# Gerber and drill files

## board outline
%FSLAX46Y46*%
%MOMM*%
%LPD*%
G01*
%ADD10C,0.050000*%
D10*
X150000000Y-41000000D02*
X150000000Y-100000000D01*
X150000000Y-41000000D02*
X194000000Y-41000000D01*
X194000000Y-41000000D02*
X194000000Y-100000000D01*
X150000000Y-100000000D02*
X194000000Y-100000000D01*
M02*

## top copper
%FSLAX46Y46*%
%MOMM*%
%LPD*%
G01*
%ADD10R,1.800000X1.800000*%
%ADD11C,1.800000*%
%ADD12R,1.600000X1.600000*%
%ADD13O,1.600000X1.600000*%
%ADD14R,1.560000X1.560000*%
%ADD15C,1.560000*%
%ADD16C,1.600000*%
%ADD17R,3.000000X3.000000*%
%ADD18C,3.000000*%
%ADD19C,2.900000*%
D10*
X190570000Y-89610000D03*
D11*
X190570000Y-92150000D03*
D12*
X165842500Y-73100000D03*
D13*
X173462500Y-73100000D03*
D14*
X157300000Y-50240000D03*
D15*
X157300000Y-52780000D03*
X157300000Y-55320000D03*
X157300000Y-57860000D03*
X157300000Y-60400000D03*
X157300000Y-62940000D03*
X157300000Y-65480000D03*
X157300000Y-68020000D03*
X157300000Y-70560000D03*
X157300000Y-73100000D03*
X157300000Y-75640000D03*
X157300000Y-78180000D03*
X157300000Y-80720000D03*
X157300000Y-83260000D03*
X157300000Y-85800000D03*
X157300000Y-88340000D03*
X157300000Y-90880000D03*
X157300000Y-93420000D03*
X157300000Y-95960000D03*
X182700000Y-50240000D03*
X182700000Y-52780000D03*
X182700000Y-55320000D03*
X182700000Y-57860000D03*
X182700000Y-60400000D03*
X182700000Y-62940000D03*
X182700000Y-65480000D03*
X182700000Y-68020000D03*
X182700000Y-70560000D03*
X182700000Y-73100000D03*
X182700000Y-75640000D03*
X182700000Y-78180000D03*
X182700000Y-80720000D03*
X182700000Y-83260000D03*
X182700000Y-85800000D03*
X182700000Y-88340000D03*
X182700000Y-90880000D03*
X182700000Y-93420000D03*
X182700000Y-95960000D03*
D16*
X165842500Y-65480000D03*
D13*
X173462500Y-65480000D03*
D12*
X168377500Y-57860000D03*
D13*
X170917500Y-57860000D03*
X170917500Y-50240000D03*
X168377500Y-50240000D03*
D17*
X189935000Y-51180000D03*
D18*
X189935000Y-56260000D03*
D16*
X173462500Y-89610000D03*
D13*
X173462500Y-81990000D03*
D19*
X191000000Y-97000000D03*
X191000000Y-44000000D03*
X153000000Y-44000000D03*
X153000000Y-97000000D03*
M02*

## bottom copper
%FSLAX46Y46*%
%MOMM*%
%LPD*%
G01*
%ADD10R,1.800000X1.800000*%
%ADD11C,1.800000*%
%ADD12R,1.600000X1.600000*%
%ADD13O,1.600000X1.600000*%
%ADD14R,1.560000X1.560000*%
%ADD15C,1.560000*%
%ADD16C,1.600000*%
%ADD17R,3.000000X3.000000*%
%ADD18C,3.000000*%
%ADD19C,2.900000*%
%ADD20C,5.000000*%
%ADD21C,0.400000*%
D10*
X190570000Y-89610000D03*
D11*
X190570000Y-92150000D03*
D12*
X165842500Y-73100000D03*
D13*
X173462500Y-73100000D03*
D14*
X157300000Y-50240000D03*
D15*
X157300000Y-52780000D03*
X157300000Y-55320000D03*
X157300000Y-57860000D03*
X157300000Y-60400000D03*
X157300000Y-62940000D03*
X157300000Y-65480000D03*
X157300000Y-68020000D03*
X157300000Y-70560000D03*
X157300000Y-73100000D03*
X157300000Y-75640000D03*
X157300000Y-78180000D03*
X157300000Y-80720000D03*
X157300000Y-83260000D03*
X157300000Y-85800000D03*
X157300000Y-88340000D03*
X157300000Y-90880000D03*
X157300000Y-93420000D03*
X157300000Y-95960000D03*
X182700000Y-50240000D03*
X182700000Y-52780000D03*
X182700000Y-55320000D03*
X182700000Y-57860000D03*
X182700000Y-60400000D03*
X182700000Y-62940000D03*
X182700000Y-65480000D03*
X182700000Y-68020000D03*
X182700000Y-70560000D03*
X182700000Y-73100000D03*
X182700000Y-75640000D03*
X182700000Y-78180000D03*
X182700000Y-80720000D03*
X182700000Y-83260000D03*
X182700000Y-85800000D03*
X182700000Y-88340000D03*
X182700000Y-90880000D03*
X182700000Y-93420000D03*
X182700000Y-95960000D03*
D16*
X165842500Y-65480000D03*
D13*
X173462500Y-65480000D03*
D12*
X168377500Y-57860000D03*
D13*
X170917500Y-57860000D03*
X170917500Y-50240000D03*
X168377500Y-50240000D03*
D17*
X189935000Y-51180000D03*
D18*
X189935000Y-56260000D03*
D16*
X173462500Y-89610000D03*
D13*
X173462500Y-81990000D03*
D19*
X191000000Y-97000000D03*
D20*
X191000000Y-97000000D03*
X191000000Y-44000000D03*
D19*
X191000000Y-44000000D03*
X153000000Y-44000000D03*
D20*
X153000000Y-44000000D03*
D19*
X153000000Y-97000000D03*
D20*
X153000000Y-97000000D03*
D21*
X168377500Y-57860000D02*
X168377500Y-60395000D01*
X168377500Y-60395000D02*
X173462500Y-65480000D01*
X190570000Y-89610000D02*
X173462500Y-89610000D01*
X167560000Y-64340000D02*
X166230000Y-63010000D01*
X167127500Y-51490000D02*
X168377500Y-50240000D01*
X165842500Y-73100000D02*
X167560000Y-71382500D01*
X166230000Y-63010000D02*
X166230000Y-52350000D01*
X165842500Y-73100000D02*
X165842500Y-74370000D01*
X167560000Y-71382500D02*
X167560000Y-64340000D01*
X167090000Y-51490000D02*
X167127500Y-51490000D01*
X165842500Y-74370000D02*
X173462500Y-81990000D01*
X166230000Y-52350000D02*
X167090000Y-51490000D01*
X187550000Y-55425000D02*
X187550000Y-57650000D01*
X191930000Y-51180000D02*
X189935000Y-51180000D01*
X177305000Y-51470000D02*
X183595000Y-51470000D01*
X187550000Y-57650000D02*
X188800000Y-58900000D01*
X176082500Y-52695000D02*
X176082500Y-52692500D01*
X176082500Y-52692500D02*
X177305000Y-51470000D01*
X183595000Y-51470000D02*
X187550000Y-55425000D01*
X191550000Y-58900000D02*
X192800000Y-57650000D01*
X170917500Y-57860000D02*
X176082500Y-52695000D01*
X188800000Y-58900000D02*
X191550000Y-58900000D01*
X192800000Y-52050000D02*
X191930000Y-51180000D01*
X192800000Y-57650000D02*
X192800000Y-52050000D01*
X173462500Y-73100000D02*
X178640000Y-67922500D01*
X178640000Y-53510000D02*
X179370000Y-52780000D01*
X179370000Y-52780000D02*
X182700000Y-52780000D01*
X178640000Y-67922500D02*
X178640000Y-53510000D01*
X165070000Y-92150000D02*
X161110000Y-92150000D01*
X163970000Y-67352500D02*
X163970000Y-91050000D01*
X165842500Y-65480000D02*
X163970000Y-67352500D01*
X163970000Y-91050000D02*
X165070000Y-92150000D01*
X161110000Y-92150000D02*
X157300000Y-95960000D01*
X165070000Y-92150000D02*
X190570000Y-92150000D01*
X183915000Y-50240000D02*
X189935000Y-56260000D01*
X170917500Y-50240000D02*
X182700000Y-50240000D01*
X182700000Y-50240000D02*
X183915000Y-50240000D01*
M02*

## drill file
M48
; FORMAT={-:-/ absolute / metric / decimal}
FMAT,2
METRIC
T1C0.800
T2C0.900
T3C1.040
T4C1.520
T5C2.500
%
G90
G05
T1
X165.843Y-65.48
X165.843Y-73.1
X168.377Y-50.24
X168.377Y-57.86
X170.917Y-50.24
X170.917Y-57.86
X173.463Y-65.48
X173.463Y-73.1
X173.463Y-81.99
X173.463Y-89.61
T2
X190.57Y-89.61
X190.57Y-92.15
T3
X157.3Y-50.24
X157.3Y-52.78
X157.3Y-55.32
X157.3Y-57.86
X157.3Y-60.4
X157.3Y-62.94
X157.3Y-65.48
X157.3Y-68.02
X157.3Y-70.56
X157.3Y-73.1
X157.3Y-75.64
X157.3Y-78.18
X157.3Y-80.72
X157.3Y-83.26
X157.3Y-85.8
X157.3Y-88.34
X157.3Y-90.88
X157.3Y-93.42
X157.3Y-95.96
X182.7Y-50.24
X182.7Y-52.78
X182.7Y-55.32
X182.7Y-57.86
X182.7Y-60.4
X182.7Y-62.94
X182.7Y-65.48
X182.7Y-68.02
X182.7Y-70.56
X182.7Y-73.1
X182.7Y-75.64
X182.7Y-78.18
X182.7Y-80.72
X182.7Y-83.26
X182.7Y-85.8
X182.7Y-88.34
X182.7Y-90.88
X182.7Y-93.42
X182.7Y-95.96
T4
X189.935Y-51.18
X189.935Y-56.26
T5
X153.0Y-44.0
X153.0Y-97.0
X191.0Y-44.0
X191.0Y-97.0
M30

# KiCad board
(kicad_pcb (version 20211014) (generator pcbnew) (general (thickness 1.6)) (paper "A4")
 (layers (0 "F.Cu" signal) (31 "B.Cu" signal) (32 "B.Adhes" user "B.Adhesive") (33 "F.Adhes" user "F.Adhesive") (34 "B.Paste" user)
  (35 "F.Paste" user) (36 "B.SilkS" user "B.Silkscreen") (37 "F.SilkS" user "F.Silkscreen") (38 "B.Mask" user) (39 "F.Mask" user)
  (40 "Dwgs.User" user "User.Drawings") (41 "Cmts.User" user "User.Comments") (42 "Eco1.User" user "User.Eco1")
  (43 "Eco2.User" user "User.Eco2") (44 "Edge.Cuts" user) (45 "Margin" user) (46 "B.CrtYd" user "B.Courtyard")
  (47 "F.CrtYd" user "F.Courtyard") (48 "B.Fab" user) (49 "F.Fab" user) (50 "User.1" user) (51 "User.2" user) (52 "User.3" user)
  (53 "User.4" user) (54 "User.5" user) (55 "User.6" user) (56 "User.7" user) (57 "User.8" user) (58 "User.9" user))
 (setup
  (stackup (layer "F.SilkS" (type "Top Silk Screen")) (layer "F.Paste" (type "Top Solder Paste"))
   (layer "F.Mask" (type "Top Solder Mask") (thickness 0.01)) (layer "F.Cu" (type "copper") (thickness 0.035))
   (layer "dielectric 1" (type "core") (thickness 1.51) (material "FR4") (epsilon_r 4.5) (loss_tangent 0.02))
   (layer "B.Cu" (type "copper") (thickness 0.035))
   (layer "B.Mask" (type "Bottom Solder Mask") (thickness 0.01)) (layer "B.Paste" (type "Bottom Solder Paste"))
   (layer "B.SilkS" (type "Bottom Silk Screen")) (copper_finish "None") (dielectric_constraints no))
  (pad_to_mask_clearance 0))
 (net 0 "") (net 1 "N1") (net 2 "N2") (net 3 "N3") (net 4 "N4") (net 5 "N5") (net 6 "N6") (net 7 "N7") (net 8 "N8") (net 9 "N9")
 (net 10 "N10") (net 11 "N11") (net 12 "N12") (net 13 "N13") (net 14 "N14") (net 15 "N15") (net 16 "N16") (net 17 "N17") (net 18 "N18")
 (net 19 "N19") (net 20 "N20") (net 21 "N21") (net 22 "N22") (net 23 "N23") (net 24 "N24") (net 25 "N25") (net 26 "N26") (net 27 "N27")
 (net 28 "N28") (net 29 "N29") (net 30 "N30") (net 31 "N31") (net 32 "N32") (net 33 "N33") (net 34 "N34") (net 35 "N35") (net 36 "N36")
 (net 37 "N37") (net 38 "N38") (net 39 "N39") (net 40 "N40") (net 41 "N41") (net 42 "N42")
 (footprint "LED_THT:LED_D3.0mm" (layer "F.Cu") (at 190.57 89.61 -90)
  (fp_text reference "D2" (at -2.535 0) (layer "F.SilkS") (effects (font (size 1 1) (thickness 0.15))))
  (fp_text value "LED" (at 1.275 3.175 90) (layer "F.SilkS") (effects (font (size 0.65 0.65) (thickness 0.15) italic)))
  (pad "1" thru_hole rect (at 0 0 270) (size 1.8 1.8) (drill 0.9) (layers *.Cu *.Mask) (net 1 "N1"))
  (pad "2" thru_hole circle (at 2.54 0 270) (size 1.8 1.8) (drill 0.9) (layers *.Cu *.Mask) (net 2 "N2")))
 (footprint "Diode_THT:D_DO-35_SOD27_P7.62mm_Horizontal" (layer "F.Cu") (at 165.8425 73.1)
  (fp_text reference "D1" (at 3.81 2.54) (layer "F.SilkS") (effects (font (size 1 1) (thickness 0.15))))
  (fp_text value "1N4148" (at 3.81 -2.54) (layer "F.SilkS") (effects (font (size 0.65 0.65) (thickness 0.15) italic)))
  (pad "1" thru_hole rect (at 0 0) (size 1.6 1.6) (drill 0.8) (layers *.Cu *.Mask) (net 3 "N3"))
  (pad "2" thru_hole oval (at 7.62 0) (size 1.6 1.6) (drill 0.8) (layers *.Cu *.Mask) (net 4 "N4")))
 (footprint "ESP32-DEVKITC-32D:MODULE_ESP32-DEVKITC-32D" (layer "F.Cu") (at 170 70)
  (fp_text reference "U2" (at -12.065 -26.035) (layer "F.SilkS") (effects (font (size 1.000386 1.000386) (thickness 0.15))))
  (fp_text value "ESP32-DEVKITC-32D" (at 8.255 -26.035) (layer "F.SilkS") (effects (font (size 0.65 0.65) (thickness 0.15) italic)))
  (pad "1" thru_hole rect locked (at -12.7 -19.76) (size 1.56 1.56) (drill 1.04) (layers *.Cu *.Mask) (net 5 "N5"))
  (pad "2" thru_hole circle locked (at -12.7 -17.22) (size 1.56 1.56) (drill 1.04) (layers *.Cu *.Mask) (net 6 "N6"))
  (pad "3" thru_hole circle locked (at -12.7 -14.68) (size 1.56 1.56) (drill 1.04) (layers *.Cu *.Mask) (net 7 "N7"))
  (pad "4" thru_hole circle locked (at -12.7 -12.14) (size 1.56 1.56) (drill 1.04) (layers *.Cu *.Mask) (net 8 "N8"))
  (pad "5" thru_hole circle locked (at -12.7 -9.6) (size 1.56 1.56) (drill 1.04) (layers *.Cu *.Mask) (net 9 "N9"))
  (pad "6" thru_hole circle locked (at -12.7 -7.06) (size 1.56 1.56) (drill 1.04) (layers *.Cu *.Mask) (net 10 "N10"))
  (pad "7" thru_hole circle locked (at -12.7 -4.52) (size 1.56 1.56) (drill 1.04) (layers *.Cu *.Mask) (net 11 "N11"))
  (pad "8" thru_hole circle locked (at -12.7 -1.98) (size 1.56 1.56) (drill 1.04) (layers *.Cu *.Mask) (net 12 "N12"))
  (pad "9" thru_hole circle locked (at -12.7 0.56) (size 1.56 1.56) (drill 1.04) (layers *.Cu *.Mask) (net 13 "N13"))
  (pad "10" thru_hole circle locked (at -12.7 3.1) (size 1.56 1.56) (drill 1.04) (layers *.Cu *.Mask) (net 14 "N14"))
  (pad "11" thru_hole circle locked (at -12.7 5.64) (size 1.56 1.56) (drill 1.04) (layers *.Cu *.Mask) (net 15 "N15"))
  (pad "12" thru_hole circle locked (at -12.7 8.18) (size 1.56 1.56) (drill 1.04) (layers *.Cu *.Mask) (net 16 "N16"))
  (pad "13" thru_hole circle locked (at -12.7 10.72) (size 1.56 1.56) (drill 1.04) (layers *.Cu *.Mask) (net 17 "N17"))
  (pad "14" thru_hole circle locked (at -12.7 13.26) (size 1.56 1.56) (drill 1.04) (layers *.Cu *.Mask) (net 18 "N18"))
  (pad "15" thru_hole circle locked (at -12.7 15.8) (size 1.56 1.56) (drill 1.04) (layers *.Cu *.Mask) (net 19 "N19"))
  (pad "16" thru_hole circle locked (at -12.7 18.34) (size 1.56 1.56) (drill 1.04) (layers *.Cu *.Mask) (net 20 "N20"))
  (pad "17" thru_hole circle locked (at -12.7 20.88) (size 1.56 1.56) (drill 1.04) (layers *.Cu *.Mask) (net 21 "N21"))
  (pad "18" thru_hole circle locked (at -12.7 23.42) (size 1.56 1.56) (drill 1.04) (layers *.Cu *.Mask) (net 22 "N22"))
  (pad "19" thru_hole circle locked (at -12.7 25.96) (size 1.56 1.56) (drill 1.04) (layers *.Cu *.Mask) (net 2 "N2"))
  (pad "20" thru_hole circle locked (at 12.7 -19.76) (size 1.56 1.56) (drill 1.04) (layers *.Cu *.Mask) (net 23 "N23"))
  (pad "21" thru_hole circle locked (at 12.7 -17.22) (size 1.56 1.56) (drill 1.04) (layers *.Cu *.Mask) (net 4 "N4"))
  (pad "22" thru_hole circle locked (at 12.7 -14.68) (size 1.56 1.56) (drill 1.04) (layers *.Cu *.Mask) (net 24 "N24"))
  (pad "23" thru_hole circle locked (at 12.7 -12.14) (size 1.56 1.56) (drill 1.04) (layers *.Cu *.Mask) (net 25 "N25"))
  (pad "24" thru_hole circle locked (at 12.7 -9.6) (size 1.56 1.56) (drill 1.04) (layers *.Cu *.Mask) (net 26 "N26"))
  (pad "25" thru_hole circle locked (at 12.7 -7.06) (size 1.56 1.56) (drill 1.04) (layers *.Cu *.Mask) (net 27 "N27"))
  (pad "26" thru_hole circle locked (at 12.7 -4.52) (size 1.56 1.56) (drill 1.04) (layers *.Cu *.Mask) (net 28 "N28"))
  (pad "27" thru_hole circle locked (at 12.7 -1.98) (size 1.56 1.56) (drill 1.04) (layers *.Cu *.Mask) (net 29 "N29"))
  (pad "28" thru_hole circle locked (at 12.7 0.56) (size 1.56 1.56) (drill 1.04) (layers *.Cu *.Mask) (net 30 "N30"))
  (pad "29" thru_hole circle locked (at 12.7 3.1) (size 1.56 1.56) (drill 1.04) (layers *.Cu *.Mask) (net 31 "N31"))
  (pad "30" thru_hole circle locked (at 12.7 5.64) (size 1.56 1.56) (drill 1.04) (layers *.Cu *.Mask) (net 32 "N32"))
  (pad "31" thru_hole circle locked (at 12.7 8.18) (size 1.56 1.56) (drill 1.04) (layers *.Cu *.Mask) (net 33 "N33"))
  (pad "32" thru_hole circle locked (at 12.7 10.72) (size 1.56 1.56) (drill 1.04) (layers *.Cu *.Mask) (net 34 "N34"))
  (pad "33" thru_hole circle locked (at 12.7 13.26) (size 1.56 1.56) (drill 1.04) (layers *.Cu *.Mask) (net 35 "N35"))
  (pad "34" thru_hole circle locked (at 12.7 15.8) (size 1.56 1.56) (drill 1.04) (layers *.Cu *.Mask) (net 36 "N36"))
  (pad "35" thru_hole circle locked (at 12.7 18.34) (size 1.56 1.56) (drill 1.04) (layers *.Cu *.Mask) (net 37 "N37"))
  (pad "36" thru_hole circle locked (at 12.7 20.88) (size 1.56 1.56) (drill 1.04) (layers *.Cu *.Mask) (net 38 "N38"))
  (pad "37" thru_hole circle locked (at 12.7 23.42) (size 1.56 1.56) (drill 1.04) (layers *.Cu *.Mask) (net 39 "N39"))
  (pad "38" thru_hole circle locked (at 12.7 25.96) (size 1.56 1.56) (drill 1.04) (layers *.Cu *.Mask) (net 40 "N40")))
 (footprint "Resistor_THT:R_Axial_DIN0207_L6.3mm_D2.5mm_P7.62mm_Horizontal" (layer "F.Cu") (at 165.8425 65.48)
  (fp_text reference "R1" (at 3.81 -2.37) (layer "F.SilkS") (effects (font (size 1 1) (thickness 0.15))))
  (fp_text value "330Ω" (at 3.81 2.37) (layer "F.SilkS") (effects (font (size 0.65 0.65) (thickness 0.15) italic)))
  (pad "1" thru_hole circle (at 0 0) (size 1.6 1.6) (drill 0.8) (layers *.Cu *.Mask) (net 2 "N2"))
  (pad "2" thru_hole oval (at 7.62 0) (size 1.6 1.6) (drill 0.8) (layers *.Cu *.Mask) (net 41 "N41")))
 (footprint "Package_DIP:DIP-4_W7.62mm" (layer "F.Cu") (at 168.3775 57.86 90)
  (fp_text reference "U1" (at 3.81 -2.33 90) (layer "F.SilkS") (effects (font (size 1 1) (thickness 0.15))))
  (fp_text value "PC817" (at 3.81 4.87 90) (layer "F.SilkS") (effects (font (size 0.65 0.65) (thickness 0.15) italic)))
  (pad "1" thru_hole rect (at 0 0 90) (size 1.6 1.6) (drill 0.8) (layers *.Cu *.Mask) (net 41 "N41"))
  (pad "2" thru_hole oval (at 0 2.54 90) (size 1.6 1.6) (drill 0.8) (layers *.Cu *.Mask) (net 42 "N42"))
  (pad "3" thru_hole oval (at 7.62 2.54 90) (size 1.6 1.6) (drill 0.8) (layers *.Cu *.Mask) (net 23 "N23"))
  (pad "4" thru_hole oval (at 7.62 0 90) (size 1.6 1.6) (drill 0.8) (layers *.Cu *.Mask) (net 3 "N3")))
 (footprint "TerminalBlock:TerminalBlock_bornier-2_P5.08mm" (layer "F.Cu") (at 189.935 51.18 -90)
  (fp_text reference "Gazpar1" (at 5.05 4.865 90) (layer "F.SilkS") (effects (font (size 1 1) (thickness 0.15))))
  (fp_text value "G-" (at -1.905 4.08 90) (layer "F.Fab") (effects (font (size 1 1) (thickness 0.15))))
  (pad "1" thru_hole rect (at 0 0 270) (size 3 3) (drill 1.52) (layers *.Cu *.Mask) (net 42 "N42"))
  (pad "2" thru_hole circle (at 5.08 0 270) (size 3 3) (drill 1.52) (layers *.Cu *.Mask) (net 23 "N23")))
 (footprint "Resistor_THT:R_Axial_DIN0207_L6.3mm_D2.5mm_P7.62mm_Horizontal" (layer "F.Cu") (at 173.4625 89.61 90)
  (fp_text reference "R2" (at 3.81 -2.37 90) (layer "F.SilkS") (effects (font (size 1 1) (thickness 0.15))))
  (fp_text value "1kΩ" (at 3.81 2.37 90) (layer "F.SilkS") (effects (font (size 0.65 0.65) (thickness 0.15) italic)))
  (pad "1" thru_hole circle (at 0 0 90) (size 1.6 1.6) (drill 0.8) (layers *.Cu *.Mask) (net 1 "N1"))
  (pad "2" thru_hole oval (at 7.62 0 90) (size 1.6 1.6) (drill 0.8) (layers *.Cu *.Mask) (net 3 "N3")))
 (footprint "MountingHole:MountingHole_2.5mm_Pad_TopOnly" (layer "B.Cu") (at 191 97 180)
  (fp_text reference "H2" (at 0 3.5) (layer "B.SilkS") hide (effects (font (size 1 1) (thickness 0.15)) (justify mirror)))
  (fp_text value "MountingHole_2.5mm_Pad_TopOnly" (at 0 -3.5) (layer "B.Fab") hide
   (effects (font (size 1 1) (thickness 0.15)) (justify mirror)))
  (pad "1" thru_hole circle (at 0 0 180) (size 2.9 2.9) (drill 2.5) (layers *.Cu *.Mask))
  (pad "1" connect circle (at 0 0 180) (size 5 5) (layers "B.Cu" "B.Mask")))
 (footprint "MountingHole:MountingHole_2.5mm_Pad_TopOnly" (layer "B.Cu") (at 191 44 180)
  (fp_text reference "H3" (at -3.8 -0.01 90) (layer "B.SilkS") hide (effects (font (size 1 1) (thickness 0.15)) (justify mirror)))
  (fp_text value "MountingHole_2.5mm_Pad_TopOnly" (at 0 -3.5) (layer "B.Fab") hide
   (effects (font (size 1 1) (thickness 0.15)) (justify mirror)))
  (pad "1" connect circle (at 0 0 180) (size 5 5) (layers "B.Cu" "B.Mask"))
  (pad "1" thru_hole circle (at 0 0 180) (size 2.9 2.9) (drill 2.5) (layers *.Cu *.Mask)))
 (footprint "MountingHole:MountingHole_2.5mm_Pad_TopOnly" (layer "B.Cu") (at 153 44 180)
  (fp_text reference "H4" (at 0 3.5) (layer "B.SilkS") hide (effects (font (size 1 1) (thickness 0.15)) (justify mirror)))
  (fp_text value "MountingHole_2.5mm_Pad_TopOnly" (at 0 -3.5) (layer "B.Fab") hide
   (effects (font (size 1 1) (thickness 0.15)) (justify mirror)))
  (pad "1" thru_hole circle (at 0 0 180) (size 2.9 2.9) (drill 2.5) (layers *.Cu *.Mask))
  (pad "1" connect circle (at 0 0 180) (size 5 5) (layers "B.Cu" "B.Mask")))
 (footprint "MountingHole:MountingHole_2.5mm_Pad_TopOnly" (layer "B.Cu") (at 153 97 180)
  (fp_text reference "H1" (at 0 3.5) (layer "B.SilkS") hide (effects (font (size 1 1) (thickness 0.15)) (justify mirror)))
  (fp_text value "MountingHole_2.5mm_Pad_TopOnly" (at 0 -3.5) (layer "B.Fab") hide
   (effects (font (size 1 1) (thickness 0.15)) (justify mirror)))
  (pad "1" thru_hole circle (at 0 0 180) (size 2.9 2.9) (drill 2.5) (layers *.Cu *.Mask))
  (pad "1" connect circle (at 0 0 180) (size 5 5) (layers "B.Cu" "B.Mask")))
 (gr_line locked (start 150 41) (end 150 100) (layer "Edge.Cuts") (width 0.05))
 (gr_line locked (start 150 41) (end 194 41) (layer "Edge.Cuts") (width 0.05))
 (gr_line locked (start 194 41) (end 194 100) (layer "Edge.Cuts") (width 0.05))
 (gr_line (start 150 100) (end 194 100) (layer "Edge.Cuts") (width 0.05))
 (segment (start 168.3775 57.86) (end 168.3775 60.395) (width 0.4) (layer "B.Cu") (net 41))
 (segment (start 168.3775 60.395) (end 173.4625 65.48) (width 0.4) (layer "B.Cu") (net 41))
 (segment (start 190.57 89.61) (end 173.4625 89.61) (width 0.4) (layer "B.Cu") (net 1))
 (segment (start 167.56 64.34) (end 166.23 63.01) (width 0.4) (layer "B.Cu") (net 3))
 (segment (start 167.1275 51.49) (end 168.3775 50.24) (width 0.4) (layer "B.Cu") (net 3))
 (segment (start 165.8425 73.1) (end 167.56 71.3825) (width 0.4) (layer "B.Cu") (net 3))
 (segment (start 166.23 63.01) (end 166.23 52.35) (width 0.4) (layer "B.Cu") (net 3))
 (segment (start 165.8425 73.1) (end 165.8425 74.37) (width 0.4) (layer "B.Cu") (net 3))
 (segment (start 167.56 71.3825) (end 167.56 64.34) (width 0.4) (layer "B.Cu") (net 3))
 (segment (start 167.09 51.49) (end 167.1275 51.49) (width 0.4) (layer "B.Cu") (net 3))
 (segment (start 165.8425 74.37) (end 173.4625 81.99) (width 0.4) (layer "B.Cu") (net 3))
 (segment (start 166.23 52.35) (end 167.09 51.49) (width 0.4) (layer "B.Cu") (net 3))
 (segment (start 187.55 55.425) (end 187.55 57.65) (width 0.4) (layer "B.Cu") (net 42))
 (segment (start 191.93 51.18) (end 189.935 51.18) (width 0.4) (layer "B.Cu") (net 42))
 (segment (start 177.305 51.47) (end 183.595 51.47) (width 0.4) (layer "B.Cu") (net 42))
 (segment (start 187.55 57.65) (end 188.8 58.9) (width 0.4) (layer "B.Cu") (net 42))
 (segment (start 176.0825 52.695) (end 176.0825 52.6925) (width 0.4) (layer "B.Cu") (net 42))
 (segment (start 176.0825 52.6925) (end 177.305 51.47) (width 0.4) (layer "B.Cu") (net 42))
 (segment (start 183.595 51.47) (end 187.55 55.425) (width 0.4) (layer "B.Cu") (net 42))
 (segment (start 191.55 58.9) (end 192.8 57.65) (width 0.4) (layer "B.Cu") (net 42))
 (segment (start 170.9175 57.86) (end 176.0825 52.695) (width 0.4) (layer "B.Cu") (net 42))
 (segment (start 188.8 58.9) (end 191.55 58.9) (width 0.4) (layer "B.Cu") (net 42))
 (segment (start 192.8 52.05) (end 191.93 51.18) (width 0.4) (layer "B.Cu") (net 42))
 (segment (start 192.8 57.65) (end 192.8 52.05) (width 0.4) (layer "B.Cu") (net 42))
 (segment (start 173.4625 73.1) (end 178.64 67.9225) (width 0.4) (layer "B.Cu") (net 4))
 (segment (start 178.64 53.51) (end 179.37 52.78) (width 0.4) (layer "B.Cu") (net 4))
 (segment (start 179.37 52.78) (end 182.7 52.78) (width 0.4) (layer "B.Cu") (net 4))
 (segment (start 178.64 67.9225) (end 178.64 53.51) (width 0.4) (layer "B.Cu") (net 4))
 (segment (start 165.07 92.15) (end 161.11 92.15) (width 0.4) (layer "B.Cu") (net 2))
 (segment (start 163.97 67.3525) (end 163.97 91.05) (width 0.4) (layer "B.Cu") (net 2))
 (segment (start 165.8425 65.48) (end 163.97 67.3525) (width 0.4) (layer "B.Cu") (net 2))
 (segment (start 163.97 91.05) (end 165.07 92.15) (width 0.4) (layer "B.Cu") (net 2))
 (segment (start 161.11 92.15) (end 157.3 95.96) (width 0.4) (layer "B.Cu") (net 2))
 (segment (start 165.07 92.15) (end 190.57 92.15) (width 0.4) (layer "B.Cu") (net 2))
 (segment (start 183.915 50.24) (end 189.935 56.26) (width 0.4) (layer "B.Cu") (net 23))
 (segment (start 170.9175 50.24) (end 182.7 50.24) (width 0.4) (layer "B.Cu") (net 23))
 (segment (start 182.7 50.24) (end 183.915 50.24) (width 0.4) (layer "B.Cu") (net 23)))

